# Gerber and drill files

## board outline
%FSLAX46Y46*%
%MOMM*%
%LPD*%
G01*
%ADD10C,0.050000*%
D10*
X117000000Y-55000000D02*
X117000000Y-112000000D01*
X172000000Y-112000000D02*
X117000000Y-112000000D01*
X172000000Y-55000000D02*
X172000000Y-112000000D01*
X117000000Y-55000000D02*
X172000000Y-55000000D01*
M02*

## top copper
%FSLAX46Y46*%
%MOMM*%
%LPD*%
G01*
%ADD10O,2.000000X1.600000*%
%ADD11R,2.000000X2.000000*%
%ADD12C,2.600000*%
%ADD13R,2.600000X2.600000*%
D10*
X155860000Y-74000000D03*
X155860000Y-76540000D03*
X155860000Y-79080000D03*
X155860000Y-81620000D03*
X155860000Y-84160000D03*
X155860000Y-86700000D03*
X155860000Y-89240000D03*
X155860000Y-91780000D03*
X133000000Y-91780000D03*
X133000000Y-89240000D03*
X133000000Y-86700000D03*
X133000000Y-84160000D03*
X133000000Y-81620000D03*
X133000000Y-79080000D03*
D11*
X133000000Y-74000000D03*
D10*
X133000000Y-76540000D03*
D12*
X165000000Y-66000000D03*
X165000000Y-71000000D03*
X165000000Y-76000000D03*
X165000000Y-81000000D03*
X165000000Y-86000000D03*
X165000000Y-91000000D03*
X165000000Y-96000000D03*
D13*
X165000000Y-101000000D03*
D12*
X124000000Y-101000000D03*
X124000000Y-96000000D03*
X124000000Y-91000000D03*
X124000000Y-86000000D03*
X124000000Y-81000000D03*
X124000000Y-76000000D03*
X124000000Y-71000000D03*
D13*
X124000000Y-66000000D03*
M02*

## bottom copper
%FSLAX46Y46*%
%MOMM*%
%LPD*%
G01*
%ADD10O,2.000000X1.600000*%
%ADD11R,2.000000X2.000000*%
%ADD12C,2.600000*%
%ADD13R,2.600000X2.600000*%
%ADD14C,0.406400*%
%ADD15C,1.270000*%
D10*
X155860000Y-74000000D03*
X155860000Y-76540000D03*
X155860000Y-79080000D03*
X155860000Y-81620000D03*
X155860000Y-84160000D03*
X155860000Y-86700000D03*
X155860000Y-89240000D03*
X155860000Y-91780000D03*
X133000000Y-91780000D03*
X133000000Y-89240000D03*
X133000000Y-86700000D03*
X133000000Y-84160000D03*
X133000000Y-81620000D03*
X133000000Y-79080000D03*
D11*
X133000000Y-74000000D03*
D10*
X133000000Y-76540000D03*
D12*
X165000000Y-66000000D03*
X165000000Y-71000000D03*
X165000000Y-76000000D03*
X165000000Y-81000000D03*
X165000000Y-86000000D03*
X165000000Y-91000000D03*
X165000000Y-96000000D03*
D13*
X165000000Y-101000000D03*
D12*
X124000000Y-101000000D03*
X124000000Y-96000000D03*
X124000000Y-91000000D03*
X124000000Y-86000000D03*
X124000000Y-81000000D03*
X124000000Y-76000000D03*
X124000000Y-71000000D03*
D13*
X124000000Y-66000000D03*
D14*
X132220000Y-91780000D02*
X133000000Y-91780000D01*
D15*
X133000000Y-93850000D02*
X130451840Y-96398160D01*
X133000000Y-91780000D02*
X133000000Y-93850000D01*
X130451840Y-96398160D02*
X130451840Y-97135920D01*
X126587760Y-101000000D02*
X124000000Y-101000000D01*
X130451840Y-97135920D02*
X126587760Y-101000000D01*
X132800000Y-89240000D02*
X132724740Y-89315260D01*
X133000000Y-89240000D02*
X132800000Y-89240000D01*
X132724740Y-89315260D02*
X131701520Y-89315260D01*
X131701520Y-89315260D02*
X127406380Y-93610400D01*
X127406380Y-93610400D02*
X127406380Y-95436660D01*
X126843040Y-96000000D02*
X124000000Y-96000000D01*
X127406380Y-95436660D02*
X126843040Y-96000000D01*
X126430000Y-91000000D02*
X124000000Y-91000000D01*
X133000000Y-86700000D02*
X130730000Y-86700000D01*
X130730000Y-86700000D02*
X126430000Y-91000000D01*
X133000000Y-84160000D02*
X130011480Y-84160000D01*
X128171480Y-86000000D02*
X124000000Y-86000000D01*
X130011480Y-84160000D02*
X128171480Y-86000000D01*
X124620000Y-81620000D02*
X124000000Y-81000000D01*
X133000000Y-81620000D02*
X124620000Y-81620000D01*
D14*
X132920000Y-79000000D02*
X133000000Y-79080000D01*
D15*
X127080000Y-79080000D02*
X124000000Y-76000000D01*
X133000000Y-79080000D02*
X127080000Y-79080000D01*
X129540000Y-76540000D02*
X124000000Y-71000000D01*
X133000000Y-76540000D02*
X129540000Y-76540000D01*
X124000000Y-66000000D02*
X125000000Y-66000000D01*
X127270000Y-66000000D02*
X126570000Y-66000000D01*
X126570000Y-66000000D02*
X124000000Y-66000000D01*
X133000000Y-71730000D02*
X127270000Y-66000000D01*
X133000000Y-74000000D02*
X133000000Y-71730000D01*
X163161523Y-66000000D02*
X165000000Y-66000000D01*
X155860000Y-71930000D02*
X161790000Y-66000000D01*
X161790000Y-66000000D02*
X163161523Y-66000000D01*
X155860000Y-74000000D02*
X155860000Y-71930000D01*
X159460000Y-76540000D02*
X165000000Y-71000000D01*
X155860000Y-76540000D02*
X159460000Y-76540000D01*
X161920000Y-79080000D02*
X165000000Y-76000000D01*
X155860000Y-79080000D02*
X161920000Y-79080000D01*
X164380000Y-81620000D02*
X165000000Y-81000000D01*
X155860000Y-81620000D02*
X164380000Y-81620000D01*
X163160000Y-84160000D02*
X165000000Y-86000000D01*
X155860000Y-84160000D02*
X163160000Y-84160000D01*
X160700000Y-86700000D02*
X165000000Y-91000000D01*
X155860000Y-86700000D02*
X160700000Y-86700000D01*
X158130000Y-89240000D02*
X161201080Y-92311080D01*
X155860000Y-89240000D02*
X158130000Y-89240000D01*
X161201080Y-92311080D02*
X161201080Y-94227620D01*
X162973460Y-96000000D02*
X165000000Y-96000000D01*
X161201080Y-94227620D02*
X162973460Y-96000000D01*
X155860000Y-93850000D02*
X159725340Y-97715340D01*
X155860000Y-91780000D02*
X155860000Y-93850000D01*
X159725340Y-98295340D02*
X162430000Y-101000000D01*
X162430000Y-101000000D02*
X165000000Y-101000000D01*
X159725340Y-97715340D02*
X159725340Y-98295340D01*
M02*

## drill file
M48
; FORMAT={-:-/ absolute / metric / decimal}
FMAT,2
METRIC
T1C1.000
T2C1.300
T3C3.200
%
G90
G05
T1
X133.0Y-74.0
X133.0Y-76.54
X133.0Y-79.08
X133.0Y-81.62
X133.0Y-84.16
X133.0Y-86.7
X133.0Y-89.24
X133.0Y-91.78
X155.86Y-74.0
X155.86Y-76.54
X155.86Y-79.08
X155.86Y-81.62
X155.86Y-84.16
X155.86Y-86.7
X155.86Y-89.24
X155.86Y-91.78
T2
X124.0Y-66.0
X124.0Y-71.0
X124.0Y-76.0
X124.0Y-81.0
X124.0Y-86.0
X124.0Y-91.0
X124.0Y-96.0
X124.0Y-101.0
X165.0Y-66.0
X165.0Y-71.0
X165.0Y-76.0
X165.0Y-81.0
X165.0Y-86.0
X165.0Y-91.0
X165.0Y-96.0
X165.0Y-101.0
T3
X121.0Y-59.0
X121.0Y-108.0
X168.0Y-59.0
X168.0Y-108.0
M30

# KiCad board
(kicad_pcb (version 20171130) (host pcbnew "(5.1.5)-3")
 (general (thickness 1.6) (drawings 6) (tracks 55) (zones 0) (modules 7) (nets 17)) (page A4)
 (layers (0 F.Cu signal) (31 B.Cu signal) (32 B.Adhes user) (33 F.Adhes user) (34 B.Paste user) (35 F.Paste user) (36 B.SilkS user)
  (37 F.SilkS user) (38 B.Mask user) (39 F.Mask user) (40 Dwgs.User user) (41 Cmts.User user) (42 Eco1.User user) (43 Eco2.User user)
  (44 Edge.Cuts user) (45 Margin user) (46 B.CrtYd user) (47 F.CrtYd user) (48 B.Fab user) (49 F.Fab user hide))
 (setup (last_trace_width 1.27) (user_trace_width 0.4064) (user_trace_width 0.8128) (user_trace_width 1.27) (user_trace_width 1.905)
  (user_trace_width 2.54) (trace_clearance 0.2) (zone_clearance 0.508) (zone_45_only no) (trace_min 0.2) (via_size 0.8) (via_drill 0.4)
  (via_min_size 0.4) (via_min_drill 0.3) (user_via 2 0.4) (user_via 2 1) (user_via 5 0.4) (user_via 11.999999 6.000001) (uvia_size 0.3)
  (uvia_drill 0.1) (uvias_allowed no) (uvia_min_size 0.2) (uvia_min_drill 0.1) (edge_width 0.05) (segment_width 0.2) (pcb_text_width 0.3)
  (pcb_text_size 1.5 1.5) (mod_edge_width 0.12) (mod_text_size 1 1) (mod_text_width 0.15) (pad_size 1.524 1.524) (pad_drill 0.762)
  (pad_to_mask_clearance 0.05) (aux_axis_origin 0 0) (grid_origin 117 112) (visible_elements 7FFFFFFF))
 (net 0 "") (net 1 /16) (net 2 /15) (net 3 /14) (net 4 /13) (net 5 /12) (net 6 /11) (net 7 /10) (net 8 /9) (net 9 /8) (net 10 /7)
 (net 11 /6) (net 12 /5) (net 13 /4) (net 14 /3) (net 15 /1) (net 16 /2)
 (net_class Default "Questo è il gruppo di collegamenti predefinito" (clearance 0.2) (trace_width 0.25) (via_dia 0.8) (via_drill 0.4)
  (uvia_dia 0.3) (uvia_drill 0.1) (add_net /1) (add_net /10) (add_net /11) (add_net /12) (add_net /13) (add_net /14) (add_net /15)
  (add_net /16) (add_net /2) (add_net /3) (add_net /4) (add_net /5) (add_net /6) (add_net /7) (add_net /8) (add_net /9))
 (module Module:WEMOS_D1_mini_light (layer F.Cu) (at 133 74)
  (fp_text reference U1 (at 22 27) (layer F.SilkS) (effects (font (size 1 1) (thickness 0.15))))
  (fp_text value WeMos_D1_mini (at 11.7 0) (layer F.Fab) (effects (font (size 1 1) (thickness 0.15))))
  (pad 16 thru_hole oval (at 22.86 0) (size 2 1.6) (drill 1) (layers *.Cu *.Mask) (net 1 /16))
  (pad 15 thru_hole oval (at 22.86 2.54) (size 2 1.6) (drill 1) (layers *.Cu *.Mask) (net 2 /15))
  (pad 14 thru_hole oval (at 22.86 5.08) (size 2 1.6) (drill 1) (layers *.Cu *.Mask) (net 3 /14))
  (pad 13 thru_hole oval (at 22.86 7.62) (size 2 1.6) (drill 1) (layers *.Cu *.Mask) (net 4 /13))
  (pad 12 thru_hole oval (at 22.86 10.16) (size 2 1.6) (drill 1) (layers *.Cu *.Mask) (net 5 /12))
  (pad 11 thru_hole oval (at 22.86 12.7) (size 2 1.6) (drill 1) (layers *.Cu *.Mask) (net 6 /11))
  (pad 10 thru_hole oval (at 22.86 15.24) (size 2 1.6) (drill 1) (layers *.Cu *.Mask) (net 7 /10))
  (pad 9 thru_hole oval (at 22.86 17.78) (size 2 1.6) (drill 1) (layers *.Cu *.Mask) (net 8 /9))
  (pad 8 thru_hole oval (at 0 17.78) (size 2 1.6) (drill 1) (layers *.Cu *.Mask) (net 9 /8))
  (pad 7 thru_hole oval (at 0 15.24) (size 2 1.6) (drill 1) (layers *.Cu *.Mask) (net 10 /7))
  (pad 6 thru_hole oval (at 0 12.7) (size 2 1.6) (drill 1) (layers *.Cu *.Mask) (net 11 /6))
  (pad 5 thru_hole oval (at 0 10.16) (size 2 1.6) (drill 1) (layers *.Cu *.Mask) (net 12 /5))
  (pad 4 thru_hole oval (at 0 7.62) (size 2 1.6) (drill 1) (layers *.Cu *.Mask) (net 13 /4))
  (pad 3 thru_hole oval (at 0 5.08) (size 2 1.6) (drill 1) (layers *.Cu *.Mask) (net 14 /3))
  (pad 1 thru_hole rect (at 0 0) (size 2 2) (drill 1) (layers *.Cu *.Mask) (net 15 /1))
  (pad 2 thru_hole oval (at 0 2.54) (size 2 1.6) (drill 1) (layers *.Cu *.Mask) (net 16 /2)))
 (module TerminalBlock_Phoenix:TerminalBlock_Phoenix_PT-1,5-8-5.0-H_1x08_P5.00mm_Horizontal (layer F.Cu) (at 165 101 90)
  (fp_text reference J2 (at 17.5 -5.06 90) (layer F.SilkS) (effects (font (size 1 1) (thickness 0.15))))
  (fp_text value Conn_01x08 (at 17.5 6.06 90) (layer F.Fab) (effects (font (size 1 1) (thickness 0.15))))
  (pad 8 thru_hole circle (at 35 0 90) (size 2.6 2.6) (drill 1.3) (layers *.Cu *.Mask) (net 1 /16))
  (pad 7 thru_hole circle (at 30 0 90) (size 2.6 2.6) (drill 1.3) (layers *.Cu *.Mask) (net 2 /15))
  (pad 6 thru_hole circle (at 25 0 90) (size 2.6 2.6) (drill 1.3) (layers *.Cu *.Mask) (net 3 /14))
  (pad 5 thru_hole circle (at 20 0 90) (size 2.6 2.6) (drill 1.3) (layers *.Cu *.Mask) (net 4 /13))
  (pad 4 thru_hole circle (at 15 0 90) (size 2.6 2.6) (drill 1.3) (layers *.Cu *.Mask) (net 5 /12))
  (pad 3 thru_hole circle (at 10 0 90) (size 2.6 2.6) (drill 1.3) (layers *.Cu *.Mask) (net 6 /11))
  (pad 2 thru_hole circle (at 5 0 90) (size 2.6 2.6) (drill 1.3) (layers *.Cu *.Mask) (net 7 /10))
  (pad 1 thru_hole rect (at 0 0 90) (size 2.6 2.6) (drill 1.3) (layers *.Cu *.Mask) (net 8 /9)))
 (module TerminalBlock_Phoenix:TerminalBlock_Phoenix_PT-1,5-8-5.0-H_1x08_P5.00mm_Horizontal (layer F.Cu) (at 124 66 270)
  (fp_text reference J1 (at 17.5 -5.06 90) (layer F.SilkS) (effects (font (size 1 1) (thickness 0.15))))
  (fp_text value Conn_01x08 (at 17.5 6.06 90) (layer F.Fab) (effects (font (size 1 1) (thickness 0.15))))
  (pad 8 thru_hole circle (at 35 0 270) (size 2.6 2.6) (drill 1.3) (layers *.Cu *.Mask) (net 9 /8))
  (pad 7 thru_hole circle (at 30 0 270) (size 2.6 2.6) (drill 1.3) (layers *.Cu *.Mask) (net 10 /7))
  (pad 6 thru_hole circle (at 25 0 270) (size 2.6 2.6) (drill 1.3) (layers *.Cu *.Mask) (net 11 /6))
  (pad 5 thru_hole circle (at 20 0 270) (size 2.6 2.6) (drill 1.3) (layers *.Cu *.Mask) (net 12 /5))
  (pad 4 thru_hole circle (at 15 0 270) (size 2.6 2.6) (drill 1.3) (layers *.Cu *.Mask) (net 13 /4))
  (pad 3 thru_hole circle (at 10 0 270) (size 2.6 2.6) (drill 1.3) (layers *.Cu *.Mask) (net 14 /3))
  (pad 2 thru_hole circle (at 5 0 270) (size 2.6 2.6) (drill 1.3) (layers *.Cu *.Mask) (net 16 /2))
  (pad 1 thru_hole rect (at 0 0 270) (size 2.6 2.6) (drill 1.3) (layers *.Cu *.Mask) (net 15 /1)))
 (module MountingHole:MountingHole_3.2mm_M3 (layer F.Cu) (at 168 108)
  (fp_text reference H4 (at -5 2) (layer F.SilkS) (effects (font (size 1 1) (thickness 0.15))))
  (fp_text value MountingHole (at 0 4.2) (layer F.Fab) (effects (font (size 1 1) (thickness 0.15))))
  (pad 1 np_thru_hole circle (at 0 0) (size 3.2 3.2) (drill 3.2) (layers *.Cu *.Mask)))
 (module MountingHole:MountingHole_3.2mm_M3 (layer F.Cu) (at 121 108)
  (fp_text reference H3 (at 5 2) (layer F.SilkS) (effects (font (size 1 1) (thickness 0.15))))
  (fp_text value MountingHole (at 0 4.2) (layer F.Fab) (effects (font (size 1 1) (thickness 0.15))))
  (pad 1 np_thru_hole circle (at 0 0) (size 3.2 3.2) (drill 3.2) (layers *.Cu *.Mask)))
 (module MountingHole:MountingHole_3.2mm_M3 (layer F.Cu) (at 168 59)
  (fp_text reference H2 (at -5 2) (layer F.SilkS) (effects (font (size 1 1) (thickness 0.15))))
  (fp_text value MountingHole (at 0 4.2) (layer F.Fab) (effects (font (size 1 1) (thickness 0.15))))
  (pad 1 np_thru_hole circle (at 0 0) (size 3.2 3.2) (drill 3.2) (layers *.Cu *.Mask)))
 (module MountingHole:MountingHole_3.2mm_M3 (layer F.Cu) (at 121 59)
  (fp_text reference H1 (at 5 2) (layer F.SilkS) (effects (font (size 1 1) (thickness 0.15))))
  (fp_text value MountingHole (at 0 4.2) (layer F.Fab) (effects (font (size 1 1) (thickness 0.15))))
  (pad 1 np_thru_hole circle (at 0 0) (size 3.2 3.2) (drill 3.2) (layers *.Cu *.Mask)))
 (gr_line (start 117 55) (end 117 112) (layer Edge.Cuts) (width 0.05))
 (gr_line (start 172 112) (end 117 112) (layer Edge.Cuts) (width 0.05))
 (gr_line (start 172 55) (end 172 112) (layer Edge.Cuts) (width 0.05))
 (gr_line (start 117 55) (end 172 55) (layer Edge.Cuts) (width 0.05))
 (segment (start 132.22 91.78) (end 133 91.78) (width 0.4064) (layer B.Cu) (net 9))
 (segment (start 133 93.85) (end 130.45184 96.39816) (width 1.27) (layer B.Cu) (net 9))
 (segment (start 133 91.78) (end 133 93.85) (width 1.27) (layer B.Cu) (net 9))
 (segment (start 130.45184 96.39816) (end 130.45184 97.13592) (width 1.27) (layer B.Cu) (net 9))
 (segment (start 126.58776 101) (end 124 101) (width 1.27) (layer B.Cu) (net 9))
 (segment (start 130.45184 97.13592) (end 126.58776 101) (width 1.27) (layer B.Cu) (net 9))
 (segment (start 132.8 89.24) (end 132.72474 89.31526) (width 1.27) (layer B.Cu) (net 10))
 (segment (start 133 89.24) (end 132.8 89.24) (width 1.27) (layer B.Cu) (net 10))
 (segment (start 132.72474 89.31526) (end 131.70152 89.31526) (width 1.27) (layer B.Cu) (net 10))
 (segment (start 131.70152 89.31526) (end 127.40638 93.6104) (width 1.27) (layer B.Cu) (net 10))
 (segment (start 127.40638 93.6104) (end 127.40638 95.43666) (width 1.27) (layer B.Cu) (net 10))
 (segment (start 126.84304 96) (end 124 96) (width 1.27) (layer B.Cu) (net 10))
 (segment (start 127.40638 95.43666) (end 126.84304 96) (width 1.27) (layer B.Cu) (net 10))
 (segment (start 126.43 91) (end 124 91) (width 1.27) (layer B.Cu) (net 11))
 (segment (start 133 86.7) (end 130.73 86.7) (width 1.27) (layer B.Cu) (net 11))
 (segment (start 130.73 86.7) (end 126.43 91) (width 1.27) (layer B.Cu) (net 11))
 (segment (start 133 84.16) (end 130.01148 84.16) (width 1.27) (layer B.Cu) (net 12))
 (segment (start 128.17148 86) (end 124 86) (width 1.27) (layer B.Cu) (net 12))
 (segment (start 130.01148 84.16) (end 128.17148 86) (width 1.27) (layer B.Cu) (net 12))
 (segment (start 124.62 81.62) (end 124 81) (width 1.27) (layer B.Cu) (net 13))
 (segment (start 133 81.62) (end 124.62 81.62) (width 1.27) (layer B.Cu) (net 13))
 (segment (start 132.92 79) (end 133 79.08) (width 0.4064) (layer B.Cu) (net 14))
 (segment (start 127.08 79.08) (end 124 76) (width 1.27) (layer B.Cu) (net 14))
 (segment (start 133 79.08) (end 127.08 79.08) (width 1.27) (layer B.Cu) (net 14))
 (segment (start 129.54 76.54) (end 124 71) (width 1.27) (layer B.Cu) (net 16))
 (segment (start 133 76.54) (end 129.54 76.54) (width 1.27) (layer B.Cu) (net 16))
 (segment (start 124 66) (end 125 66) (width 1.27) (layer B.Cu) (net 15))
 (segment (start 127.27 66) (end 126.57 66) (width 1.27) (layer B.Cu) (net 15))
 (segment (start 126.57 66) (end 124 66) (width 1.27) (layer B.Cu) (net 15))
 (segment (start 133 71.73) (end 127.27 66) (width 1.27) (layer B.Cu) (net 15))
 (segment (start 133 74) (end 133 71.73) (width 1.27) (layer B.Cu) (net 15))
 (segment (start 163.161523 66) (end 165 66) (width 1.27) (layer B.Cu) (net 1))
 (segment (start 155.86 71.93) (end 161.79 66) (width 1.27) (layer B.Cu) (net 1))
 (segment (start 161.79 66) (end 163.161523 66) (width 1.27) (layer B.Cu) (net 1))
 (segment (start 155.86 74) (end 155.86 71.93) (width 1.27) (layer B.Cu) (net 1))
 (segment (start 159.46 76.54) (end 165 71) (width 1.27) (layer B.Cu) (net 2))
 (segment (start 155.86 76.54) (end 159.46 76.54) (width 1.27) (layer B.Cu) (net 2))
 (segment (start 161.92 79.08) (end 165 76) (width 1.27) (layer B.Cu) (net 3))
 (segment (start 155.86 79.08) (end 161.92 79.08) (width 1.27) (layer B.Cu) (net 3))
 (segment (start 164.38 81.62) (end 165 81) (width 1.27) (layer B.Cu) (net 4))
 (segment (start 155.86 81.62) (end 164.38 81.62) (width 1.27) (layer B.Cu) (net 4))
 (segment (start 163.16 84.16) (end 165 86) (width 1.27) (layer B.Cu) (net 5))
 (segment (start 155.86 84.16) (end 163.16 84.16) (width 1.27) (layer B.Cu) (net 5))
 (segment (start 160.7 86.7) (end 165 91) (width 1.27) (layer B.Cu) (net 6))
 (segment (start 155.86 86.7) (end 160.7 86.7) (width 1.27) (layer B.Cu) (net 6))
 (segment (start 158.13 89.24) (end 161.20108 92.31108) (width 1.27) (layer B.Cu) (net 7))
 (segment (start 155.86 89.24) (end 158.13 89.24) (width 1.27) (layer B.Cu) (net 7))
 (segment (start 161.20108 92.31108) (end 161.20108 94.22762) (width 1.27) (layer B.Cu) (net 7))
 (segment (start 162.97346 96) (end 165 96) (width 1.27) (layer B.Cu) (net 7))
 (segment (start 161.20108 94.22762) (end 162.97346 96) (width 1.27) (layer B.Cu) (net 7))
 (segment (start 155.86 93.85) (end 159.72534 97.71534) (width 1.27) (layer B.Cu) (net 8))
 (segment (start 155.86 91.78) (end 155.86 93.85) (width 1.27) (layer B.Cu) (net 8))
 (segment (start 159.72534 98.29534) (end 162.43 101) (width 1.27) (layer B.Cu) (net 8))
 (segment (start 162.43 101) (end 165 101) (width 1.27) (layer B.Cu) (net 8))
 (segment (start 159.72534 97.71534) (end 159.72534 98.29534) (width 1.27) (layer B.Cu) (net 8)))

